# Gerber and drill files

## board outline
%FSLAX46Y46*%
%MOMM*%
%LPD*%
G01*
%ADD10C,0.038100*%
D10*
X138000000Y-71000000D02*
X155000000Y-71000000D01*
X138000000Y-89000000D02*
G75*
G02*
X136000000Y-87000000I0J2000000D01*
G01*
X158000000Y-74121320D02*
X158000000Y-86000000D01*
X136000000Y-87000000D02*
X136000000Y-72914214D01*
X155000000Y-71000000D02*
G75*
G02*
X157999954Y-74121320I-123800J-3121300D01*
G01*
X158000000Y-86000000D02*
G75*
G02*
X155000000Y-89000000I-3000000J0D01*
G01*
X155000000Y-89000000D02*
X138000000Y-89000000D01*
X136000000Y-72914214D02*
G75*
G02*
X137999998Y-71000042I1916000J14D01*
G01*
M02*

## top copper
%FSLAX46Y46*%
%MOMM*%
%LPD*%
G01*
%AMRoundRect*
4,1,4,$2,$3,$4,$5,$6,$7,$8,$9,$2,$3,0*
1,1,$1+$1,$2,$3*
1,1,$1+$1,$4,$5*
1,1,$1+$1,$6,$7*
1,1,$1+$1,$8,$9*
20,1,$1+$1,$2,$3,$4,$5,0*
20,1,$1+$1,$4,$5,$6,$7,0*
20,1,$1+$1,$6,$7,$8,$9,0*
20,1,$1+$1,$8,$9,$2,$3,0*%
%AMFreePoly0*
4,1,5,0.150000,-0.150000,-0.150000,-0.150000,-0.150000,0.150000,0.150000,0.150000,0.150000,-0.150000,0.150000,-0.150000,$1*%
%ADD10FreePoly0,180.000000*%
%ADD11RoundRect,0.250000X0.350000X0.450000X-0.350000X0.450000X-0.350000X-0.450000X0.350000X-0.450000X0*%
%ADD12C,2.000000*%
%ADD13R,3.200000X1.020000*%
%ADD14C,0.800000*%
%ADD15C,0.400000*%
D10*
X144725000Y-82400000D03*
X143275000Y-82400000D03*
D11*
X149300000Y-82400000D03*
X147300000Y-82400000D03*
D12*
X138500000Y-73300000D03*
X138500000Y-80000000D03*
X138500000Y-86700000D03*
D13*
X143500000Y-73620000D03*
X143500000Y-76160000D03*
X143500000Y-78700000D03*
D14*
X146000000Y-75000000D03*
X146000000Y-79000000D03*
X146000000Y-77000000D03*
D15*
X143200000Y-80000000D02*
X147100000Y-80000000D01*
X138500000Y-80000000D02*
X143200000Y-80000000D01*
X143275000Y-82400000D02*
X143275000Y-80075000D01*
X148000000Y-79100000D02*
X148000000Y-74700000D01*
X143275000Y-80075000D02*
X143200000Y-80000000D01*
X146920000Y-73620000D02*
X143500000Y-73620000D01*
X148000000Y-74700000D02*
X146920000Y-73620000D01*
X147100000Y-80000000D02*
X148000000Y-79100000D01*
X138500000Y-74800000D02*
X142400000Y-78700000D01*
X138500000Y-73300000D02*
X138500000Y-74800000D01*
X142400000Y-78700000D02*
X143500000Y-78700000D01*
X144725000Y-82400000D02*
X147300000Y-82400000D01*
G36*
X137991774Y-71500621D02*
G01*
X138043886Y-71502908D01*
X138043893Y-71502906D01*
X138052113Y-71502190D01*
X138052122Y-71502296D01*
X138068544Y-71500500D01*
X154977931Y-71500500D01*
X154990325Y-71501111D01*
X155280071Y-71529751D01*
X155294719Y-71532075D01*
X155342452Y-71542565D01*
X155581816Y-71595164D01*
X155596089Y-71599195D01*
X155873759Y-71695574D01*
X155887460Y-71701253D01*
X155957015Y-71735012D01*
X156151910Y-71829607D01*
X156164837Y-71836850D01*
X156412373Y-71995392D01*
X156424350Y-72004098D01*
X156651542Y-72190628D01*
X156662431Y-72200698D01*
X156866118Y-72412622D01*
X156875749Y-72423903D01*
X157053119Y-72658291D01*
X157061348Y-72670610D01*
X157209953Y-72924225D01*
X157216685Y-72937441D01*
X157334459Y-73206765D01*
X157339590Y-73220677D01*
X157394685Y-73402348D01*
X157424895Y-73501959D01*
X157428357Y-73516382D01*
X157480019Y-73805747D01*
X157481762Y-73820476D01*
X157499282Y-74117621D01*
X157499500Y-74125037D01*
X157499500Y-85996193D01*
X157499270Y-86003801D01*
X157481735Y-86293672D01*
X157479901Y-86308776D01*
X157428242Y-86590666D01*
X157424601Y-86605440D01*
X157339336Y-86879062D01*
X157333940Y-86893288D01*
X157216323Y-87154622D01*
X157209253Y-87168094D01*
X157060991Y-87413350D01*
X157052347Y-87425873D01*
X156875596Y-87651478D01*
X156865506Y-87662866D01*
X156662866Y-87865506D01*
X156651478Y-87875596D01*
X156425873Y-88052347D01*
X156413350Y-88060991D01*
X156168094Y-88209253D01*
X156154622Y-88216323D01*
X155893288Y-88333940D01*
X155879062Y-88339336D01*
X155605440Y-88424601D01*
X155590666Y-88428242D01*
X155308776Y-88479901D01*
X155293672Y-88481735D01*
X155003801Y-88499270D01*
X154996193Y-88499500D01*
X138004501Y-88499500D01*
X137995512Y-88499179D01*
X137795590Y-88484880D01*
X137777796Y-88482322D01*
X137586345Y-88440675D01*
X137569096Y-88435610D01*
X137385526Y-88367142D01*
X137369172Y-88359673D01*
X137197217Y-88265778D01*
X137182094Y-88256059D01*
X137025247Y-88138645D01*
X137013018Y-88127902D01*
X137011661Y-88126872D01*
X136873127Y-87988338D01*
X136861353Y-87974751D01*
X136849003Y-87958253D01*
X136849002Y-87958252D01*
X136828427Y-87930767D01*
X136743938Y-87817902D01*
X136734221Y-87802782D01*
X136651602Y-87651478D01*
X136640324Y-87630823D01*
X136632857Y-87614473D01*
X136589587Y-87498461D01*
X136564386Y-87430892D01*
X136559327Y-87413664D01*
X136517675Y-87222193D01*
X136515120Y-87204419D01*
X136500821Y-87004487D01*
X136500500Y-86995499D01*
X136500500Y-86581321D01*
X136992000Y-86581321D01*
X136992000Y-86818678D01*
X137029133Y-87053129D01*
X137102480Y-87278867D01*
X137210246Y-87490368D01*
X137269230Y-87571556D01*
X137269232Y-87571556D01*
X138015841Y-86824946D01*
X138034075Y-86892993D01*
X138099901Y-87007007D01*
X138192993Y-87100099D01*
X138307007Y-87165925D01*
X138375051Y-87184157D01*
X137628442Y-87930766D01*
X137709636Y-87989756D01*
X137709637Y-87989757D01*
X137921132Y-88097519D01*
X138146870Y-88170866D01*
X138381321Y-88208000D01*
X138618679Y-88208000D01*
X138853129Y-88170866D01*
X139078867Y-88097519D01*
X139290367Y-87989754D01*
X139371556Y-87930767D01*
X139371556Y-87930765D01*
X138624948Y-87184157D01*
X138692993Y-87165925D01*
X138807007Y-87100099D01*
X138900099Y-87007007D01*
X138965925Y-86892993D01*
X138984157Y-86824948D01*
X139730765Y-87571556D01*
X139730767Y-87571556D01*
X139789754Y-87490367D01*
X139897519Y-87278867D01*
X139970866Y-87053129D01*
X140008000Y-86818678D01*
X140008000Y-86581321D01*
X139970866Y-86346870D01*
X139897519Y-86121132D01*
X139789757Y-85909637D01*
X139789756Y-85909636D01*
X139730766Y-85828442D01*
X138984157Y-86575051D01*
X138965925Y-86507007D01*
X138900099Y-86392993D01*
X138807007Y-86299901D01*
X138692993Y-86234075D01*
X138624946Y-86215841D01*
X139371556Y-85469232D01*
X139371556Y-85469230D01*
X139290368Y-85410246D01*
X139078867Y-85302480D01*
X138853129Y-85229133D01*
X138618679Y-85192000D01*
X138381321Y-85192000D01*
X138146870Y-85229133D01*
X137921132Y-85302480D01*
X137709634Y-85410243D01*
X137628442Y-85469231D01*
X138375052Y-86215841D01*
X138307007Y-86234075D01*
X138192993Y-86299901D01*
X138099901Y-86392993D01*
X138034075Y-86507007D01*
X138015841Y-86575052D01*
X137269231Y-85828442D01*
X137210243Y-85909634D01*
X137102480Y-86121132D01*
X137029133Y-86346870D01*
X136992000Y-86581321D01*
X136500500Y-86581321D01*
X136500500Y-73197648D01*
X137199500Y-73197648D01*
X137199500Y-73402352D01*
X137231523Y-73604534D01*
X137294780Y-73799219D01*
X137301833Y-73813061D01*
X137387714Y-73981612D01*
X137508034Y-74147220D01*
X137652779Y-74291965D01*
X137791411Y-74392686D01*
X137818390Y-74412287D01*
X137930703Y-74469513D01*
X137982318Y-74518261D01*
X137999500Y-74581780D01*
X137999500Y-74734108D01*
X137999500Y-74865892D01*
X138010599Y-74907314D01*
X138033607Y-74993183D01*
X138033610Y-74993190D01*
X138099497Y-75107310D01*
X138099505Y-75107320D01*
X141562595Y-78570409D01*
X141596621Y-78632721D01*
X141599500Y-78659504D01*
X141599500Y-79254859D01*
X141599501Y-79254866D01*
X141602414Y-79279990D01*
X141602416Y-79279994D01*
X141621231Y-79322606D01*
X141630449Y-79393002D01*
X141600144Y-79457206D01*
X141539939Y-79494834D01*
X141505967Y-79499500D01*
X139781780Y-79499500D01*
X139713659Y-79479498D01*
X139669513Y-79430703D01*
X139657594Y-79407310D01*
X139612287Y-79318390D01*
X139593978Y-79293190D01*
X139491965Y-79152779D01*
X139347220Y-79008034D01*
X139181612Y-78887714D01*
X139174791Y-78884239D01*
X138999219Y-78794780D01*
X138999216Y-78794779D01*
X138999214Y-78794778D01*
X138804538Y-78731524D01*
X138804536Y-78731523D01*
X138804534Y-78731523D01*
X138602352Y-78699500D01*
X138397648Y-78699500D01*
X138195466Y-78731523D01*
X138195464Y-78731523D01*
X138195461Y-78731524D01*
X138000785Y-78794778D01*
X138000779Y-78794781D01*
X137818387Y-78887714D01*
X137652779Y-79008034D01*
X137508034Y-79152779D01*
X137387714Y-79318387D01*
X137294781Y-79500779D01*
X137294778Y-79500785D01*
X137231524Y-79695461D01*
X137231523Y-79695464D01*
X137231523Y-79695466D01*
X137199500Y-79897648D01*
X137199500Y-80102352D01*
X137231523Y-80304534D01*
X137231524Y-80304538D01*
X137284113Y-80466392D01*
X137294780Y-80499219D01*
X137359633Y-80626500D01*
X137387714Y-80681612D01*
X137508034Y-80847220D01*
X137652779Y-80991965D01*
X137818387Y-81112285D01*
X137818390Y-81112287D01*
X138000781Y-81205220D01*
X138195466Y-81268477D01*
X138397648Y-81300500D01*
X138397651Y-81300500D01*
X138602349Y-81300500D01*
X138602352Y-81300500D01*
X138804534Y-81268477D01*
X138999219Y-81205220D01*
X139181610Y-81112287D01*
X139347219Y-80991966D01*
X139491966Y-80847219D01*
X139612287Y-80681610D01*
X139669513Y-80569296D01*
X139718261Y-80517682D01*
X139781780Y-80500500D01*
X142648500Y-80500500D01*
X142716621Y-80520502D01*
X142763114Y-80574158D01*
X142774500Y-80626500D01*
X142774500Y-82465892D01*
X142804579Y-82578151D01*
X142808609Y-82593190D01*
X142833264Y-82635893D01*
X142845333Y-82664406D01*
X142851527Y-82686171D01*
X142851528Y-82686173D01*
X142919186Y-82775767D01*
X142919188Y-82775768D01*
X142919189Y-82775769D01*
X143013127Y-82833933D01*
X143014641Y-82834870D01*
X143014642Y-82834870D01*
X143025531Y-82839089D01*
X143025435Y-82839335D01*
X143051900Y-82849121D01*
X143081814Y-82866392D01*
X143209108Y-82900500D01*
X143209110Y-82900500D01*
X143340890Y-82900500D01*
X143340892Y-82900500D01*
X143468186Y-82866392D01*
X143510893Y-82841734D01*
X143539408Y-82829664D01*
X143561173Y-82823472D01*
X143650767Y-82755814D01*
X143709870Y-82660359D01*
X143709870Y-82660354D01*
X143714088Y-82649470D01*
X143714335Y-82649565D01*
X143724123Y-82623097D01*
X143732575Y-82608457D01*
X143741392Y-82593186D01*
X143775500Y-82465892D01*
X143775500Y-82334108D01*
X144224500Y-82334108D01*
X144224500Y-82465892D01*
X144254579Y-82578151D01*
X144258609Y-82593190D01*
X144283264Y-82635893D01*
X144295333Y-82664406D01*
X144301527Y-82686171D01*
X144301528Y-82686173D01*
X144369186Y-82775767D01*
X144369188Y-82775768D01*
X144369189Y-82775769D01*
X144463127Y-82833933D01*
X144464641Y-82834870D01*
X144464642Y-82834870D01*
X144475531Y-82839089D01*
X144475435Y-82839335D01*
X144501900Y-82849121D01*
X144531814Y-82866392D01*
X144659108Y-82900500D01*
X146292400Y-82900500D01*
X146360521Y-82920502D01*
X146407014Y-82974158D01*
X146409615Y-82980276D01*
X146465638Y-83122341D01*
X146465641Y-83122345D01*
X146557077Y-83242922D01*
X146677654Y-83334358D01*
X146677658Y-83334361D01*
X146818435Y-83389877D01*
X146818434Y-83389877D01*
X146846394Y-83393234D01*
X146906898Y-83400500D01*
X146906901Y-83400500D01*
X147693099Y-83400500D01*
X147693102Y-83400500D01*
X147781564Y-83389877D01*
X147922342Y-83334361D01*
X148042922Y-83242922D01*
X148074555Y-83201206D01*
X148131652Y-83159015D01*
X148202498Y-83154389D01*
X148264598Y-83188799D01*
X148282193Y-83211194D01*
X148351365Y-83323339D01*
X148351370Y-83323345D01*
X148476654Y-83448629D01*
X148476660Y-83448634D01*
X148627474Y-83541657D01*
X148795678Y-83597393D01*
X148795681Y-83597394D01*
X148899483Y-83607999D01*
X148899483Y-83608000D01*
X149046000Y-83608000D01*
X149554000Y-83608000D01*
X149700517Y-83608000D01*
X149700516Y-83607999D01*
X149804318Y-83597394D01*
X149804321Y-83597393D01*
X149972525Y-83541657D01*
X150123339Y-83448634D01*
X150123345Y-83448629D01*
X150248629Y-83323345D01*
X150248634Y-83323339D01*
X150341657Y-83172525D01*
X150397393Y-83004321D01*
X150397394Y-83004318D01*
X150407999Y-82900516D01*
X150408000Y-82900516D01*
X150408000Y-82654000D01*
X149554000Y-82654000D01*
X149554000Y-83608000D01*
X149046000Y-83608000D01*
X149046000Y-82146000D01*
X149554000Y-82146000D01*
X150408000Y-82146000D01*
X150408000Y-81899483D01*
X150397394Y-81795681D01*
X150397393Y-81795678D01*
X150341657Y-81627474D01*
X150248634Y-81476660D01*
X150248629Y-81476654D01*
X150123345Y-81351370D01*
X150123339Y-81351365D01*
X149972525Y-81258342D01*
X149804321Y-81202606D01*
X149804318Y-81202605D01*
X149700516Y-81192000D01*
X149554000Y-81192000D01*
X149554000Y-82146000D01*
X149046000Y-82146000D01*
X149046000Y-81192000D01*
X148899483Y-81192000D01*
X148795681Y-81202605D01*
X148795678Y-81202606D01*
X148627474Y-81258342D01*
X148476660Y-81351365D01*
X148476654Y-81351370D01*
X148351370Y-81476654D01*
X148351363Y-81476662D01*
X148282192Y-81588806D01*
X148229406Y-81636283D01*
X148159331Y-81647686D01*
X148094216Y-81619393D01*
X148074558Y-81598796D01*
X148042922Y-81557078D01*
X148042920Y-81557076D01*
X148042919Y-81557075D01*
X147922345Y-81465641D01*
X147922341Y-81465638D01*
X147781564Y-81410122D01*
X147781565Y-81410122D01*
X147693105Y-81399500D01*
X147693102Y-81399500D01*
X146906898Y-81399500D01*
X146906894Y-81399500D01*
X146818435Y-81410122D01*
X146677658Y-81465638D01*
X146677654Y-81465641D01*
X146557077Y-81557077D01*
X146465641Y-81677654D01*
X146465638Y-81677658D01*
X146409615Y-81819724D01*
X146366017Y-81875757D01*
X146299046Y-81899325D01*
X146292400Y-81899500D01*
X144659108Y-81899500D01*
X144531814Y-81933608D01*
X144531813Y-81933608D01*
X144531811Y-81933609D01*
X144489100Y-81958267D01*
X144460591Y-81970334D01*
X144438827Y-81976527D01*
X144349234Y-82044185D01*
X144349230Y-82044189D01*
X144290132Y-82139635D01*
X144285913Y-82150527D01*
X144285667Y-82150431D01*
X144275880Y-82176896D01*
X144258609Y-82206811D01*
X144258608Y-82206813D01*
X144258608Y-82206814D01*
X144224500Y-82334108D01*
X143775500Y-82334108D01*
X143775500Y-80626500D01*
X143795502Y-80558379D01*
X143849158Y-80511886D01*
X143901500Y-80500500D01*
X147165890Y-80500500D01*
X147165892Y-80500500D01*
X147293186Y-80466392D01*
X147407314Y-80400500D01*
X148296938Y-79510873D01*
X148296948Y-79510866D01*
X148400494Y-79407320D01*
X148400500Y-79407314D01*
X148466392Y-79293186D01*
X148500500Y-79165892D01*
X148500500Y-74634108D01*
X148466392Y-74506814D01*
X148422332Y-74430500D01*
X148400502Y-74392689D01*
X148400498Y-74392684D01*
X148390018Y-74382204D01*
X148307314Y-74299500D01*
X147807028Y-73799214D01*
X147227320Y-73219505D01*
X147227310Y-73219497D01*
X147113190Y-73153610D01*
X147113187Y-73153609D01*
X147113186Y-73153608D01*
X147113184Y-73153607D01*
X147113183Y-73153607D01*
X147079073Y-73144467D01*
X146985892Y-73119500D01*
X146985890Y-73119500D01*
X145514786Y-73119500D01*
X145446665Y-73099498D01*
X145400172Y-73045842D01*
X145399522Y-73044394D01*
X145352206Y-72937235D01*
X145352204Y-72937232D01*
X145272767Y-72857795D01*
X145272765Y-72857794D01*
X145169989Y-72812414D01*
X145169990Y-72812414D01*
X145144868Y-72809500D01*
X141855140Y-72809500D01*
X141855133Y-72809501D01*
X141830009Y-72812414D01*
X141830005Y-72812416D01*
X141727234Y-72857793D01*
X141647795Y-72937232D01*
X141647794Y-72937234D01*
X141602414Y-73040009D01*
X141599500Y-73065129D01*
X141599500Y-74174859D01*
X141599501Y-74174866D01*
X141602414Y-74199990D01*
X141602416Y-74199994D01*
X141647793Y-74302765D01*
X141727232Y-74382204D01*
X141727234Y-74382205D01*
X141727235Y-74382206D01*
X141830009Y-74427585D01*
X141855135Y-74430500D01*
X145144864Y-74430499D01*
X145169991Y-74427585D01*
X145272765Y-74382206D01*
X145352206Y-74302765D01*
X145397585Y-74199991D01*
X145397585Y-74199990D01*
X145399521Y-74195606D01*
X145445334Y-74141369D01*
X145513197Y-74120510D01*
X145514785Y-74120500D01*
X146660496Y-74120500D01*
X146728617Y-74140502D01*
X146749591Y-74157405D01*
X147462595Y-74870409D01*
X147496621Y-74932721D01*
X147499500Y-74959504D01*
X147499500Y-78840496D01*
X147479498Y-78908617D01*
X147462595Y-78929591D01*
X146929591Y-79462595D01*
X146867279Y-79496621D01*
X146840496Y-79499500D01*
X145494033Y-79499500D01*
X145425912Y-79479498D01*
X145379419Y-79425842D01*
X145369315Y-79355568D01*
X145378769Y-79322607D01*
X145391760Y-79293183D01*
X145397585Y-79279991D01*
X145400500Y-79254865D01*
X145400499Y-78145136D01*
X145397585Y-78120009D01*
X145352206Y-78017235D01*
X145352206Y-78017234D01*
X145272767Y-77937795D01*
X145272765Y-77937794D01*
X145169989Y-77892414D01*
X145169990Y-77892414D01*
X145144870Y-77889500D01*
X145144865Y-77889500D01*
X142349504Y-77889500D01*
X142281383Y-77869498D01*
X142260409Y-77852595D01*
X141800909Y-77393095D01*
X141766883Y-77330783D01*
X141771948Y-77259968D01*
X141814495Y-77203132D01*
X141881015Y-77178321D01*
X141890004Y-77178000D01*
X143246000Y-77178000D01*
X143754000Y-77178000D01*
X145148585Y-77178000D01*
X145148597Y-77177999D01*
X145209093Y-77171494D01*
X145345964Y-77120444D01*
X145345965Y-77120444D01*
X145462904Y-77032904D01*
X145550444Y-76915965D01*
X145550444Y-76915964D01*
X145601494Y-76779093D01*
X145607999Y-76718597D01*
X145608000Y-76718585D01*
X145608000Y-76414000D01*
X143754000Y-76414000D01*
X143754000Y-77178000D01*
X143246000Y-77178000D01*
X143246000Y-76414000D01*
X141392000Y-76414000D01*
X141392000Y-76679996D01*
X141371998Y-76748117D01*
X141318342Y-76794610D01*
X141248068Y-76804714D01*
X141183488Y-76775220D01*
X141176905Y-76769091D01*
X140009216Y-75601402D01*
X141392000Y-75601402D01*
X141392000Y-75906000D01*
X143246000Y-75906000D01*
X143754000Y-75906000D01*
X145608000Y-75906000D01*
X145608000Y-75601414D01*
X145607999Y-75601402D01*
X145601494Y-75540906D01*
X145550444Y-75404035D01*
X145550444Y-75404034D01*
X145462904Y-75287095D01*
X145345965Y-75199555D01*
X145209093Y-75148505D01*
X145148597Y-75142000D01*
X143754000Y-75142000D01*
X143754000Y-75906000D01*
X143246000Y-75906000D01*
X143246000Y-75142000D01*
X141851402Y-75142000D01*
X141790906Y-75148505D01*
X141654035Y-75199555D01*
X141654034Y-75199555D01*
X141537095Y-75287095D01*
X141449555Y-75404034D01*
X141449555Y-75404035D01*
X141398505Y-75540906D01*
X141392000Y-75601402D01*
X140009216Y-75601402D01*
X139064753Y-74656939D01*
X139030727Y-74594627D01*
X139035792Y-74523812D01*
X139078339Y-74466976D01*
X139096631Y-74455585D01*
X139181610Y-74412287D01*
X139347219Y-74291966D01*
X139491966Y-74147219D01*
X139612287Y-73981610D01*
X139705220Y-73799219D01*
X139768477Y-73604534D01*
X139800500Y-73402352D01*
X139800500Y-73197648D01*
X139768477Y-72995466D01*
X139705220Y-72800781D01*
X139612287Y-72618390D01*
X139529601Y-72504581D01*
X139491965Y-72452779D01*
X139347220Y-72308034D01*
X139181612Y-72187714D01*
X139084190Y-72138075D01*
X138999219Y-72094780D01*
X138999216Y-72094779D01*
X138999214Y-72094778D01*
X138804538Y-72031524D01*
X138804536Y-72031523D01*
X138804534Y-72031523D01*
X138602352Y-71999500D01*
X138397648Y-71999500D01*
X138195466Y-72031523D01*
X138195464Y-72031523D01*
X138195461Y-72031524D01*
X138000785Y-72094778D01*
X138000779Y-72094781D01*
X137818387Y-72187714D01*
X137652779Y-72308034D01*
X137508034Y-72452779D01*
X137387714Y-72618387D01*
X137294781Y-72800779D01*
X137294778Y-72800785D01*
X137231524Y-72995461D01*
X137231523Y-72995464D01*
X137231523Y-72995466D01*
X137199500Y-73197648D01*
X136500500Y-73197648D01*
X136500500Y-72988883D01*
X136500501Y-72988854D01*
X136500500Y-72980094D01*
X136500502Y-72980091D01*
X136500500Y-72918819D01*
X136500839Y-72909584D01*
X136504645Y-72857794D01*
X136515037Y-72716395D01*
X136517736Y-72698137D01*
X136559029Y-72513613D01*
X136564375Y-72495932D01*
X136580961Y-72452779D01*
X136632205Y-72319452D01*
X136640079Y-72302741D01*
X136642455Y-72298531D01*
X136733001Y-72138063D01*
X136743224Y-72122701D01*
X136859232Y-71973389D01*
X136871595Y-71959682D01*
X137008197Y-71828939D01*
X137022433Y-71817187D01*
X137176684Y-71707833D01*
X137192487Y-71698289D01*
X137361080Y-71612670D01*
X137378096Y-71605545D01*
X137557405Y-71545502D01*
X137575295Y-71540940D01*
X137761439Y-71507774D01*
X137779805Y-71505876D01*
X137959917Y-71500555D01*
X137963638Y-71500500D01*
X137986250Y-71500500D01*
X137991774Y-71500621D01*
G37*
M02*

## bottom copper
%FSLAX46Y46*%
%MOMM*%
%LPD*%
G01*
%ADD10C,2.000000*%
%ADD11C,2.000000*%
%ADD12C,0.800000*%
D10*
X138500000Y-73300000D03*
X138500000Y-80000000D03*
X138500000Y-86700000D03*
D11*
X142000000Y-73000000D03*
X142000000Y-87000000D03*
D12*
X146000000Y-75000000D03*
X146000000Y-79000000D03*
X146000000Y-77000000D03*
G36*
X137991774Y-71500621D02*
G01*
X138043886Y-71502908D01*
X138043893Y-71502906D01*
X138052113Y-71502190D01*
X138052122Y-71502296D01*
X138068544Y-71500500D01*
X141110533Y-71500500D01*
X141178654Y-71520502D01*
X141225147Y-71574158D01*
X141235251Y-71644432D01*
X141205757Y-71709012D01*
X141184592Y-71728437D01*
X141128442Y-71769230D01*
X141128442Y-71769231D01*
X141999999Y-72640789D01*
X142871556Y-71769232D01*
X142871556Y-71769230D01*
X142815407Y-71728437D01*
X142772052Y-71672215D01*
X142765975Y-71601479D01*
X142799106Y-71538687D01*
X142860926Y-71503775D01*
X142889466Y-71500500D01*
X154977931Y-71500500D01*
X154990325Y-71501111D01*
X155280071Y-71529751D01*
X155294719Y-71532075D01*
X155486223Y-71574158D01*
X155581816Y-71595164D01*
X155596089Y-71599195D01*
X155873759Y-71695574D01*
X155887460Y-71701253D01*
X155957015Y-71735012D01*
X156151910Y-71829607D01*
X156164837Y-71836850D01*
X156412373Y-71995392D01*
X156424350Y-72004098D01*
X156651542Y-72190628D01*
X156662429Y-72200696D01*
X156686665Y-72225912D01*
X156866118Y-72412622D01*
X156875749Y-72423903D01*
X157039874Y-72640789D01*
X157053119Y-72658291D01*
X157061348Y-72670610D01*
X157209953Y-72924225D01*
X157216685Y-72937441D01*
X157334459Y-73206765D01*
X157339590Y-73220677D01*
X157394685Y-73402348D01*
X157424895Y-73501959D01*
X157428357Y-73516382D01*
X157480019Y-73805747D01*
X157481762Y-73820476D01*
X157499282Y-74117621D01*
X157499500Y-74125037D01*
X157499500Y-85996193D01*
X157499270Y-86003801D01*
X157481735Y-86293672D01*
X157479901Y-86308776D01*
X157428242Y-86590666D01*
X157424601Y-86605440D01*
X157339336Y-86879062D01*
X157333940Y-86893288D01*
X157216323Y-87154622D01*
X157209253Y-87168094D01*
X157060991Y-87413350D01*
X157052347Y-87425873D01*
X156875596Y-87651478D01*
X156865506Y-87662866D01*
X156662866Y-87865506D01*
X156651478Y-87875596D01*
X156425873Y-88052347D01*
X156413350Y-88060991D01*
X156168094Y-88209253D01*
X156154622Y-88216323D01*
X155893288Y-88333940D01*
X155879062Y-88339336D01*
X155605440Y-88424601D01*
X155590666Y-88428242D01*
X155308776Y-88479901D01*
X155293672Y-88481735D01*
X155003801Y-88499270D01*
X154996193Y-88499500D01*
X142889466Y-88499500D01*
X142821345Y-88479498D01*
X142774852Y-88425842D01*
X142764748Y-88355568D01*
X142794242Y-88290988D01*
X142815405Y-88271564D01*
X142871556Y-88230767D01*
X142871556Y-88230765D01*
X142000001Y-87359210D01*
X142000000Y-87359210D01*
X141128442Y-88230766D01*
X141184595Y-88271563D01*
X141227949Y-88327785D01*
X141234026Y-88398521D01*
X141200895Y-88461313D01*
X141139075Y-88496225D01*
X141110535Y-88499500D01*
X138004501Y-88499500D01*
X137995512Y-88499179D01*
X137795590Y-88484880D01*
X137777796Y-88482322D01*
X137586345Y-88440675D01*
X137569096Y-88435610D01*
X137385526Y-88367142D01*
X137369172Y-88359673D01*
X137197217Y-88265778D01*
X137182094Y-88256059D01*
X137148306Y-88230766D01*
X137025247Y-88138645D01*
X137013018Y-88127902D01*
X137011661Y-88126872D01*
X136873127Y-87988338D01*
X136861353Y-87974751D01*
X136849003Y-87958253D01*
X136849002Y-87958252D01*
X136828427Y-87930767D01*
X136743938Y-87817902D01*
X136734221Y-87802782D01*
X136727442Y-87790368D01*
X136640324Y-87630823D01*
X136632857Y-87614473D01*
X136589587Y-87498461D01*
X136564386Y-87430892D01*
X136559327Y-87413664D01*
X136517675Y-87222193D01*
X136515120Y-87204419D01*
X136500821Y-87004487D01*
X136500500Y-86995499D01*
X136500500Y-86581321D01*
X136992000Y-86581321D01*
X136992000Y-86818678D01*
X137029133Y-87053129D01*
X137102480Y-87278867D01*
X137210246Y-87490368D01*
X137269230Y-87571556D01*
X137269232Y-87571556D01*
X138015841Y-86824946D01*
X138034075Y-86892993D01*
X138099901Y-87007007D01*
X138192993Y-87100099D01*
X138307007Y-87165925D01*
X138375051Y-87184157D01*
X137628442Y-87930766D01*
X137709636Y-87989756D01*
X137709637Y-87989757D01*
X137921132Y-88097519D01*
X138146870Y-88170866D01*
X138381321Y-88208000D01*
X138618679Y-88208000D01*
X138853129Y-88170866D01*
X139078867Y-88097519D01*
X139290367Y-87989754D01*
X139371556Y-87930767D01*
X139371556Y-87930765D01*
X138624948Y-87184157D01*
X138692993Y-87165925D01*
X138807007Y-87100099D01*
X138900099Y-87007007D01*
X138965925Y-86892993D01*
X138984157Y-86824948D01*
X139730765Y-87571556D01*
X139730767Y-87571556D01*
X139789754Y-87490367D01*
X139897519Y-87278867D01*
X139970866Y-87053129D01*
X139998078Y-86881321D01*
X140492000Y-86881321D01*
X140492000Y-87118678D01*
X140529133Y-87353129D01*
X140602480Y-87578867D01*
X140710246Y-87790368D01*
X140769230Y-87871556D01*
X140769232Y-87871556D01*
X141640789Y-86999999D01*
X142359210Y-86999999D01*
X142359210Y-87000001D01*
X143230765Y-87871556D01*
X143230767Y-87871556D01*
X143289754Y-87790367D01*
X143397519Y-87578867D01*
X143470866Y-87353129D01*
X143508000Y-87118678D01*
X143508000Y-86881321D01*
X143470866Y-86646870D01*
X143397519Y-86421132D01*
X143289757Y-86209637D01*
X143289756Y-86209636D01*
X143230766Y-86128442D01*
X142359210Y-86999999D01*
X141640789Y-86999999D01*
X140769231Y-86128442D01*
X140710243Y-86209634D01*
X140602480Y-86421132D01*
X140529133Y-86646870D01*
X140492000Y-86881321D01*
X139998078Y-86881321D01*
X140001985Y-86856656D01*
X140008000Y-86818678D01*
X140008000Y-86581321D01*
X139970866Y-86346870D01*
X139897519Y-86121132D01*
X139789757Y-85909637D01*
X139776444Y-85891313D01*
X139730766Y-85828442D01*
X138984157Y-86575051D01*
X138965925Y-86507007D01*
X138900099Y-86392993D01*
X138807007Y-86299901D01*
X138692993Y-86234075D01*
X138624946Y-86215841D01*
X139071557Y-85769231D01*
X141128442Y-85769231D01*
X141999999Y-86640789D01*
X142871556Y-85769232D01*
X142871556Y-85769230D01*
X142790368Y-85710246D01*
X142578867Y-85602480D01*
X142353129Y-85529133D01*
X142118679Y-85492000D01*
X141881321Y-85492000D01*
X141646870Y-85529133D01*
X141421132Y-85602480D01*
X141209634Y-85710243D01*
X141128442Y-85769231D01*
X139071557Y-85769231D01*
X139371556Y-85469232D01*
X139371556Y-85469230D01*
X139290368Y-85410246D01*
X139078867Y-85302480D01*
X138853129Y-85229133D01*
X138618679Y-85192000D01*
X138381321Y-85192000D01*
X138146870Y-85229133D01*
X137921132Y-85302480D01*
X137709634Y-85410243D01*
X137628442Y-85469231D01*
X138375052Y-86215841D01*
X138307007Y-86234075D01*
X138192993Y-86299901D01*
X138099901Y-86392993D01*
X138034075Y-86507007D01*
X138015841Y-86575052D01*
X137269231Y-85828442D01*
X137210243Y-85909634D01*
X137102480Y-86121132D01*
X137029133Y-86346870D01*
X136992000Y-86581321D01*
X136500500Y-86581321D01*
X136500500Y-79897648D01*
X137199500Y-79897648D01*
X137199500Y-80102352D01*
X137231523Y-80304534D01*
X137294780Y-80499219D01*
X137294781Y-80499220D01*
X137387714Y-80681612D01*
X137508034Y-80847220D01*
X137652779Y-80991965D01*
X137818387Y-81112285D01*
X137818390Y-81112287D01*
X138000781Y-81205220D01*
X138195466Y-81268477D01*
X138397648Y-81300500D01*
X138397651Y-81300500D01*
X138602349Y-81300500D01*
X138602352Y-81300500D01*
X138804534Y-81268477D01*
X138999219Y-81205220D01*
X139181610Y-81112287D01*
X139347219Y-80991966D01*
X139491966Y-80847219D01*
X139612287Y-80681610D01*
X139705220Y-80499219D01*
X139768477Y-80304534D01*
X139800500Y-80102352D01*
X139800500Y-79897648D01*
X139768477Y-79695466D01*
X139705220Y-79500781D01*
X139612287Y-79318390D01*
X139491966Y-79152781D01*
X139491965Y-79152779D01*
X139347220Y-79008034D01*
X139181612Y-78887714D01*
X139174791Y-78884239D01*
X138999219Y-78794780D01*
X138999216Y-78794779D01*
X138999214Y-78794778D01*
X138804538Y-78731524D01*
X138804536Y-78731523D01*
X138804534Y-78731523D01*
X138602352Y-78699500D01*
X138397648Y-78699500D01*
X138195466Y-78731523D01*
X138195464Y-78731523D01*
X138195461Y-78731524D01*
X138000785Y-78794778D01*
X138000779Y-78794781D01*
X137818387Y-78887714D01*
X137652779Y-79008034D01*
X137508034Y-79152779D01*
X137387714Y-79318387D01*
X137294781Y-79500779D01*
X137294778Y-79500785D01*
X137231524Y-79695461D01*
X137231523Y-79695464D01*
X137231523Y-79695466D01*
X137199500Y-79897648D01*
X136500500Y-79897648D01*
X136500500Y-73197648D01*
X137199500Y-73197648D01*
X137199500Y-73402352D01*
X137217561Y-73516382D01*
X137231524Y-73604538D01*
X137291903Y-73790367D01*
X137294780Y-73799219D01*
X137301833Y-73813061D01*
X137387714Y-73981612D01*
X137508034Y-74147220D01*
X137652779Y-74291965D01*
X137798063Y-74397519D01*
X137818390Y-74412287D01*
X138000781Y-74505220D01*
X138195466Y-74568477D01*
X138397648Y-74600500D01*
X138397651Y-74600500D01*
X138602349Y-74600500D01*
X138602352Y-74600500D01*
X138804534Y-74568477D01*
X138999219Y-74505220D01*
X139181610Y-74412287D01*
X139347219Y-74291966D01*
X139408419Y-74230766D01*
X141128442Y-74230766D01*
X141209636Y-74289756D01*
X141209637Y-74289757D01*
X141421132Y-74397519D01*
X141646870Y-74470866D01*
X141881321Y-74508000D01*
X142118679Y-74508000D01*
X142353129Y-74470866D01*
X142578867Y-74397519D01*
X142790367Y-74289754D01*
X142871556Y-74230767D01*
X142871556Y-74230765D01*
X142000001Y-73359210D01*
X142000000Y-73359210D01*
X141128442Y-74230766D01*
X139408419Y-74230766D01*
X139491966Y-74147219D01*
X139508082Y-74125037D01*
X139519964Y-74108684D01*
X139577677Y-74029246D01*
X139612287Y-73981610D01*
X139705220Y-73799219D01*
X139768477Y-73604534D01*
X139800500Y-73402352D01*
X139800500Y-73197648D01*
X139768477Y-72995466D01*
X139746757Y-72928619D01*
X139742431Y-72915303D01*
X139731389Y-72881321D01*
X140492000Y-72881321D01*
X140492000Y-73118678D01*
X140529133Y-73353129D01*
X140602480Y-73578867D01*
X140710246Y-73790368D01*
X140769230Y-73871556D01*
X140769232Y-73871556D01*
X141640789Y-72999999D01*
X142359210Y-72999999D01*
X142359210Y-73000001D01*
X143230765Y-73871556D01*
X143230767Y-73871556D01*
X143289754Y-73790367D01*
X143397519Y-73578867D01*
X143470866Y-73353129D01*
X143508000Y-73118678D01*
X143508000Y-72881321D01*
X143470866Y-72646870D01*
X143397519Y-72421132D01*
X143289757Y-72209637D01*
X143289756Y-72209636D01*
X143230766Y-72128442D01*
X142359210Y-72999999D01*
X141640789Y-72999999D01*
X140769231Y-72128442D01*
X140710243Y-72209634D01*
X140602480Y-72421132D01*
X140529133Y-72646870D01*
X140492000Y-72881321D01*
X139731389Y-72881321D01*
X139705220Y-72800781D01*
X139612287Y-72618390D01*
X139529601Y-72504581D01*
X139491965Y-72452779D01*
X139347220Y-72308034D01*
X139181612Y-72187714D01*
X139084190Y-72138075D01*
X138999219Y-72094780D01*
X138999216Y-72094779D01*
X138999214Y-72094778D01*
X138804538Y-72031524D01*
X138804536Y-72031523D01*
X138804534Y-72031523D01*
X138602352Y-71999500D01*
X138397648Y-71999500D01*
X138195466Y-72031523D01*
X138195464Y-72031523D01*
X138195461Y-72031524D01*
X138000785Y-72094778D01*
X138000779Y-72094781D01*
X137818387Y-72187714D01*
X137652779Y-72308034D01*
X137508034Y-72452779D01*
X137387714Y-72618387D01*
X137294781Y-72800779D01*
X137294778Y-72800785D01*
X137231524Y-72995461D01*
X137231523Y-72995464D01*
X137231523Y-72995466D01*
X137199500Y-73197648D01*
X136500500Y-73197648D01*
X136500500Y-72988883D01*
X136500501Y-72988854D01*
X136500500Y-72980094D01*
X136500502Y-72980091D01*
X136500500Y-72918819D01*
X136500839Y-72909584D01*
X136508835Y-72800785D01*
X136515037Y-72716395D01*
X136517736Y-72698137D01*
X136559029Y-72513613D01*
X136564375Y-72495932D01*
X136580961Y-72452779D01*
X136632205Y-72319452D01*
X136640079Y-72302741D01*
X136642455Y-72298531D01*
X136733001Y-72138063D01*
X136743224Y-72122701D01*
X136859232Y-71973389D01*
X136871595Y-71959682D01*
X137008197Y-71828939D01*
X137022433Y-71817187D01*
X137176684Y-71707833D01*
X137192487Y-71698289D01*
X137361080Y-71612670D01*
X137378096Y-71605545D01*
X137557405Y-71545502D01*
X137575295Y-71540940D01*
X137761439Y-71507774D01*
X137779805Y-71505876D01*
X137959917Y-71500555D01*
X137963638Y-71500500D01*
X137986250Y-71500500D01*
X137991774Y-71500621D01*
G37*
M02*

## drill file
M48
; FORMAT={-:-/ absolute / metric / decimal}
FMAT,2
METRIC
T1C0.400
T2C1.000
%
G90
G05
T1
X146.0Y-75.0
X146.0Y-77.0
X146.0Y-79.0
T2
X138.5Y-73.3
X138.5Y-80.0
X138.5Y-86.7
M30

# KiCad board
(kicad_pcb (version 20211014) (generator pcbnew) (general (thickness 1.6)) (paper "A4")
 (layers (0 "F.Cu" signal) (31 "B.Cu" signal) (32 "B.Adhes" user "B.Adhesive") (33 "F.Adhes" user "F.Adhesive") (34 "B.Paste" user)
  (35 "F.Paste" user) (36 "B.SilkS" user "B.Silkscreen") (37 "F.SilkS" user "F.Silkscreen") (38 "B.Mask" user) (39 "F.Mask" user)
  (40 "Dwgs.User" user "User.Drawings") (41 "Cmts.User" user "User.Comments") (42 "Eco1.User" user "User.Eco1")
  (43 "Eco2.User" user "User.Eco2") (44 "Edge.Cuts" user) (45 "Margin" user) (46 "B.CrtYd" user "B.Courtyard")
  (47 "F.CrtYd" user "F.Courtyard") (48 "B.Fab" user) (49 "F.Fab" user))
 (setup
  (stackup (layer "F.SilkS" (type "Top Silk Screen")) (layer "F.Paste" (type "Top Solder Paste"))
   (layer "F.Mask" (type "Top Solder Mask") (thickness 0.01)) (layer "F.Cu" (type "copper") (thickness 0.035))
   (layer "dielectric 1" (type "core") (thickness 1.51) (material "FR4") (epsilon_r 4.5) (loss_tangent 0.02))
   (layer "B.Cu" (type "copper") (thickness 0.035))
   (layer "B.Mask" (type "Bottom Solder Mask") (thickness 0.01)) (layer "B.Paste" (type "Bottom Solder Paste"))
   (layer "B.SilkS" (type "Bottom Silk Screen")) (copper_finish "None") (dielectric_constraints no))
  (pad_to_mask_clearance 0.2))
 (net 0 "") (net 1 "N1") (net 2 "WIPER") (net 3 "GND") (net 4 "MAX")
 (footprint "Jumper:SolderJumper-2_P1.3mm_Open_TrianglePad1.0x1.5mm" (layer "F.Cu") (at 144 82.4 180)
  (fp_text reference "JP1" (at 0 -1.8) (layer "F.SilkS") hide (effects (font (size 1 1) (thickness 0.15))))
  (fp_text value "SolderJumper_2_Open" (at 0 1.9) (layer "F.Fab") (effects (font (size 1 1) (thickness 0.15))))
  (pad "1" smd custom (at -0.725 0 180) (size 0.3 0.3) (layers "F.Cu" "F.Mask") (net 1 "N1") (zone_connect 2)
   (options (clearance outline) (anchor rect)) (primitives))
  (pad "2" smd custom (at 0.725 0 180) (size 0.3 0.3) (layers "F.Cu" "F.Mask") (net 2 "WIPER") (zone_connect 2)
   (options (clearance outline) (anchor rect)) (primitives)))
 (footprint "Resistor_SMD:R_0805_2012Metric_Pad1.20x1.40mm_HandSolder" (layer "F.Cu") (at 148.3 82.4 180)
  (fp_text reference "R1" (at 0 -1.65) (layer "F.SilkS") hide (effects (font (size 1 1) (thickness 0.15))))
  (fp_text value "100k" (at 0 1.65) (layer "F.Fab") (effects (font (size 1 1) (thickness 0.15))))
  (pad "1" smd roundrect (at -1 0 180) (size 1.2 1.4) (layers "F.Cu" "F.Paste" "F.Mask") (roundrect_rratio 0.208333) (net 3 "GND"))
  (pad "2" smd roundrect (at 1 0 180) (size 1.2 1.4) (layers "F.Cu" "F.Paste" "F.Mask") (roundrect_rratio 0.208333) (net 1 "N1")))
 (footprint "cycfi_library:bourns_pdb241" (layer "F.Cu") (at 138.5 80)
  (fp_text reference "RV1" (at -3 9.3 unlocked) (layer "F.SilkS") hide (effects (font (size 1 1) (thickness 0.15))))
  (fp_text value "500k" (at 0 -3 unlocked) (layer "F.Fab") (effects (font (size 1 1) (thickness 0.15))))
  (pad "1" thru_hole circle (at 0 -6.7) (size 2 2) (drill 1) (layers *.Cu *.Mask) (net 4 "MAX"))
  (pad "2" thru_hole circle (at 0 0) (size 2 2) (drill 1) (layers *.Cu *.Mask) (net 2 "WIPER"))
  (pad "3" thru_hole circle (at 0 6.7) (size 2 2) (drill 1) (layers *.Cu *.Mask) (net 3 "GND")))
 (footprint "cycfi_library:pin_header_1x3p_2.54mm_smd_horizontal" (layer "F.Cu") (at 143.5 73.62)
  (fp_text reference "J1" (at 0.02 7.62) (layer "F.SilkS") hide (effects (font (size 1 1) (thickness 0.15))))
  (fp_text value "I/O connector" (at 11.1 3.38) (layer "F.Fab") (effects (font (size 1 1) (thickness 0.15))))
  (pad "1" smd rect (at 0 0) (size 3.2 1.02) (layers "F.Cu" "F.Paste" "F.Mask") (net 2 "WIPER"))
  (pad "2" smd rect (at 0 2.54) (size 3.2 1.02) (layers "F.Cu" "F.Paste" "F.Mask") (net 3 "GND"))
  (pad "3" smd rect (at 0 5.08) (size 3.2 1.02) (layers "F.Cu" "F.Paste" "F.Mask") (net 4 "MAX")))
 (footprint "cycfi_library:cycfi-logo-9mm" (layer "F.Cu") (at 150.7 85.7)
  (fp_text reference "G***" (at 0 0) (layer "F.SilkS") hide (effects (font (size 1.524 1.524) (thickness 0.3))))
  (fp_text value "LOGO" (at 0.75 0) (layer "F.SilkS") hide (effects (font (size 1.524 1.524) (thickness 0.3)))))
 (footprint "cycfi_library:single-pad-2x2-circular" (layer "B.Cu") (at 142 73 180)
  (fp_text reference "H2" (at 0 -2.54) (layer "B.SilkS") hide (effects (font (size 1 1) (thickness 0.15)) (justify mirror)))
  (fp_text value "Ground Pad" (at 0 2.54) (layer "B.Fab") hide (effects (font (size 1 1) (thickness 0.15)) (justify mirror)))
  (pad "1" smd circle (at 0 0 180) (size 2 2) (layers "B.Cu" "B.Paste" "B.Mask") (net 3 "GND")))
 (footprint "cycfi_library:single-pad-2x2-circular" (layer "B.Cu") (at 142 87 180)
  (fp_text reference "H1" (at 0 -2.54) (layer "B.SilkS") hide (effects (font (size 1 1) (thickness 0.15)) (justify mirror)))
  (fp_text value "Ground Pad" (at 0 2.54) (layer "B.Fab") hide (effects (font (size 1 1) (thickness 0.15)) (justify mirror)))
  (pad "1" smd circle (at 0 0 180) (size 2 2) (layers "B.Cu" "B.Paste" "B.Mask") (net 3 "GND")))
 (gr_line (start 138 71) (end 155 71) (layer "Edge.Cuts") (width 0.0381))
 (gr_arc (start 138 89) (mid 136.585786 88.414214) (end 136 87) (layer "Edge.Cuts") (width 0.0381))
 (gr_line (start 158 74.12132) (end 158 86) (layer "Edge.Cuts") (width 0.0381))
 (gr_line (start 136 87) (end 136 72.914214) (layer "Edge.Cuts") (width 0.0381))
 (gr_arc (start 155 71) (mid 157.128402 71.956683) (end 158 74.12132) (layer "Edge.Cuts") (width 0.0381))
 (gr_arc (start 158 86) (mid 157.121318 88.121318) (end 155 89) (layer "Edge.Cuts") (width 0.0381))
 (gr_line (start 155 89) (end 138 89) (layer "Edge.Cuts") (width 0.0381))
 (gr_arc (start 136 72.914214) (mid 136.591204 71.529971) (end 138 71) (layer "Edge.Cuts") (width 0.0381))
 (segment (start 143.2 80) (end 147.1 80) (width 0.4) (layer "F.Cu") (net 2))
 (segment (start 138.5 80) (end 143.2 80) (width 0.4) (layer "F.Cu") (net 2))
 (segment (start 143.275 82.4) (end 143.275 80.075) (width 0.4) (layer "F.Cu") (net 2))
 (segment (start 148 79.1) (end 148 74.7) (width 0.4) (layer "F.Cu") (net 2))
 (segment (start 143.275 80.075) (end 143.2 80) (width 0.4) (layer "F.Cu") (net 2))
 (segment (start 146.92 73.62) (end 143.5 73.62) (width 0.4) (layer "F.Cu") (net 2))
 (segment (start 148 74.7) (end 146.92 73.62) (width 0.4) (layer "F.Cu") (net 2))
 (segment (start 147.1 80) (end 148 79.1) (width 0.4) (layer "F.Cu") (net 2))
 (via (at 146 75) (size 0.8) (drill 0.4) (layers "F.Cu" "B.Cu") (free) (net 3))
 (via (at 146 79) (size 0.8) (drill 0.4) (layers "F.Cu" "B.Cu") (free) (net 3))
 (via (at 146 77) (size 0.8) (drill 0.4) (layers "F.Cu" "B.Cu") (free) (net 3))
 (segment (start 138.5 74.8) (end 142.4 78.7) (width 0.4) (layer "F.Cu") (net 4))
 (segment (start 138.5 73.3) (end 138.5 74.8) (width 0.4) (layer "F.Cu") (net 4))
 (segment (start 142.4 78.7) (end 143.5 78.7) (width 0.4) (layer "F.Cu") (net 4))
 (segment (start 144.725 82.4) (end 147.3 82.4) (width 0.4) (layer "F.Cu") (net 1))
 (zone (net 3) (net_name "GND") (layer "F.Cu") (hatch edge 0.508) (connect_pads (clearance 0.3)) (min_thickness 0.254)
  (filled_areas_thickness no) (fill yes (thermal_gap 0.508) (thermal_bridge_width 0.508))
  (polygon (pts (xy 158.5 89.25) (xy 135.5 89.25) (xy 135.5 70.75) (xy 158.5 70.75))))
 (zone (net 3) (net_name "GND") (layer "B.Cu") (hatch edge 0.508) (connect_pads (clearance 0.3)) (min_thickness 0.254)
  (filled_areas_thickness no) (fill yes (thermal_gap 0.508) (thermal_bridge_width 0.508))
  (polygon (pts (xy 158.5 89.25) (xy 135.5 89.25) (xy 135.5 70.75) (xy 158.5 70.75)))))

